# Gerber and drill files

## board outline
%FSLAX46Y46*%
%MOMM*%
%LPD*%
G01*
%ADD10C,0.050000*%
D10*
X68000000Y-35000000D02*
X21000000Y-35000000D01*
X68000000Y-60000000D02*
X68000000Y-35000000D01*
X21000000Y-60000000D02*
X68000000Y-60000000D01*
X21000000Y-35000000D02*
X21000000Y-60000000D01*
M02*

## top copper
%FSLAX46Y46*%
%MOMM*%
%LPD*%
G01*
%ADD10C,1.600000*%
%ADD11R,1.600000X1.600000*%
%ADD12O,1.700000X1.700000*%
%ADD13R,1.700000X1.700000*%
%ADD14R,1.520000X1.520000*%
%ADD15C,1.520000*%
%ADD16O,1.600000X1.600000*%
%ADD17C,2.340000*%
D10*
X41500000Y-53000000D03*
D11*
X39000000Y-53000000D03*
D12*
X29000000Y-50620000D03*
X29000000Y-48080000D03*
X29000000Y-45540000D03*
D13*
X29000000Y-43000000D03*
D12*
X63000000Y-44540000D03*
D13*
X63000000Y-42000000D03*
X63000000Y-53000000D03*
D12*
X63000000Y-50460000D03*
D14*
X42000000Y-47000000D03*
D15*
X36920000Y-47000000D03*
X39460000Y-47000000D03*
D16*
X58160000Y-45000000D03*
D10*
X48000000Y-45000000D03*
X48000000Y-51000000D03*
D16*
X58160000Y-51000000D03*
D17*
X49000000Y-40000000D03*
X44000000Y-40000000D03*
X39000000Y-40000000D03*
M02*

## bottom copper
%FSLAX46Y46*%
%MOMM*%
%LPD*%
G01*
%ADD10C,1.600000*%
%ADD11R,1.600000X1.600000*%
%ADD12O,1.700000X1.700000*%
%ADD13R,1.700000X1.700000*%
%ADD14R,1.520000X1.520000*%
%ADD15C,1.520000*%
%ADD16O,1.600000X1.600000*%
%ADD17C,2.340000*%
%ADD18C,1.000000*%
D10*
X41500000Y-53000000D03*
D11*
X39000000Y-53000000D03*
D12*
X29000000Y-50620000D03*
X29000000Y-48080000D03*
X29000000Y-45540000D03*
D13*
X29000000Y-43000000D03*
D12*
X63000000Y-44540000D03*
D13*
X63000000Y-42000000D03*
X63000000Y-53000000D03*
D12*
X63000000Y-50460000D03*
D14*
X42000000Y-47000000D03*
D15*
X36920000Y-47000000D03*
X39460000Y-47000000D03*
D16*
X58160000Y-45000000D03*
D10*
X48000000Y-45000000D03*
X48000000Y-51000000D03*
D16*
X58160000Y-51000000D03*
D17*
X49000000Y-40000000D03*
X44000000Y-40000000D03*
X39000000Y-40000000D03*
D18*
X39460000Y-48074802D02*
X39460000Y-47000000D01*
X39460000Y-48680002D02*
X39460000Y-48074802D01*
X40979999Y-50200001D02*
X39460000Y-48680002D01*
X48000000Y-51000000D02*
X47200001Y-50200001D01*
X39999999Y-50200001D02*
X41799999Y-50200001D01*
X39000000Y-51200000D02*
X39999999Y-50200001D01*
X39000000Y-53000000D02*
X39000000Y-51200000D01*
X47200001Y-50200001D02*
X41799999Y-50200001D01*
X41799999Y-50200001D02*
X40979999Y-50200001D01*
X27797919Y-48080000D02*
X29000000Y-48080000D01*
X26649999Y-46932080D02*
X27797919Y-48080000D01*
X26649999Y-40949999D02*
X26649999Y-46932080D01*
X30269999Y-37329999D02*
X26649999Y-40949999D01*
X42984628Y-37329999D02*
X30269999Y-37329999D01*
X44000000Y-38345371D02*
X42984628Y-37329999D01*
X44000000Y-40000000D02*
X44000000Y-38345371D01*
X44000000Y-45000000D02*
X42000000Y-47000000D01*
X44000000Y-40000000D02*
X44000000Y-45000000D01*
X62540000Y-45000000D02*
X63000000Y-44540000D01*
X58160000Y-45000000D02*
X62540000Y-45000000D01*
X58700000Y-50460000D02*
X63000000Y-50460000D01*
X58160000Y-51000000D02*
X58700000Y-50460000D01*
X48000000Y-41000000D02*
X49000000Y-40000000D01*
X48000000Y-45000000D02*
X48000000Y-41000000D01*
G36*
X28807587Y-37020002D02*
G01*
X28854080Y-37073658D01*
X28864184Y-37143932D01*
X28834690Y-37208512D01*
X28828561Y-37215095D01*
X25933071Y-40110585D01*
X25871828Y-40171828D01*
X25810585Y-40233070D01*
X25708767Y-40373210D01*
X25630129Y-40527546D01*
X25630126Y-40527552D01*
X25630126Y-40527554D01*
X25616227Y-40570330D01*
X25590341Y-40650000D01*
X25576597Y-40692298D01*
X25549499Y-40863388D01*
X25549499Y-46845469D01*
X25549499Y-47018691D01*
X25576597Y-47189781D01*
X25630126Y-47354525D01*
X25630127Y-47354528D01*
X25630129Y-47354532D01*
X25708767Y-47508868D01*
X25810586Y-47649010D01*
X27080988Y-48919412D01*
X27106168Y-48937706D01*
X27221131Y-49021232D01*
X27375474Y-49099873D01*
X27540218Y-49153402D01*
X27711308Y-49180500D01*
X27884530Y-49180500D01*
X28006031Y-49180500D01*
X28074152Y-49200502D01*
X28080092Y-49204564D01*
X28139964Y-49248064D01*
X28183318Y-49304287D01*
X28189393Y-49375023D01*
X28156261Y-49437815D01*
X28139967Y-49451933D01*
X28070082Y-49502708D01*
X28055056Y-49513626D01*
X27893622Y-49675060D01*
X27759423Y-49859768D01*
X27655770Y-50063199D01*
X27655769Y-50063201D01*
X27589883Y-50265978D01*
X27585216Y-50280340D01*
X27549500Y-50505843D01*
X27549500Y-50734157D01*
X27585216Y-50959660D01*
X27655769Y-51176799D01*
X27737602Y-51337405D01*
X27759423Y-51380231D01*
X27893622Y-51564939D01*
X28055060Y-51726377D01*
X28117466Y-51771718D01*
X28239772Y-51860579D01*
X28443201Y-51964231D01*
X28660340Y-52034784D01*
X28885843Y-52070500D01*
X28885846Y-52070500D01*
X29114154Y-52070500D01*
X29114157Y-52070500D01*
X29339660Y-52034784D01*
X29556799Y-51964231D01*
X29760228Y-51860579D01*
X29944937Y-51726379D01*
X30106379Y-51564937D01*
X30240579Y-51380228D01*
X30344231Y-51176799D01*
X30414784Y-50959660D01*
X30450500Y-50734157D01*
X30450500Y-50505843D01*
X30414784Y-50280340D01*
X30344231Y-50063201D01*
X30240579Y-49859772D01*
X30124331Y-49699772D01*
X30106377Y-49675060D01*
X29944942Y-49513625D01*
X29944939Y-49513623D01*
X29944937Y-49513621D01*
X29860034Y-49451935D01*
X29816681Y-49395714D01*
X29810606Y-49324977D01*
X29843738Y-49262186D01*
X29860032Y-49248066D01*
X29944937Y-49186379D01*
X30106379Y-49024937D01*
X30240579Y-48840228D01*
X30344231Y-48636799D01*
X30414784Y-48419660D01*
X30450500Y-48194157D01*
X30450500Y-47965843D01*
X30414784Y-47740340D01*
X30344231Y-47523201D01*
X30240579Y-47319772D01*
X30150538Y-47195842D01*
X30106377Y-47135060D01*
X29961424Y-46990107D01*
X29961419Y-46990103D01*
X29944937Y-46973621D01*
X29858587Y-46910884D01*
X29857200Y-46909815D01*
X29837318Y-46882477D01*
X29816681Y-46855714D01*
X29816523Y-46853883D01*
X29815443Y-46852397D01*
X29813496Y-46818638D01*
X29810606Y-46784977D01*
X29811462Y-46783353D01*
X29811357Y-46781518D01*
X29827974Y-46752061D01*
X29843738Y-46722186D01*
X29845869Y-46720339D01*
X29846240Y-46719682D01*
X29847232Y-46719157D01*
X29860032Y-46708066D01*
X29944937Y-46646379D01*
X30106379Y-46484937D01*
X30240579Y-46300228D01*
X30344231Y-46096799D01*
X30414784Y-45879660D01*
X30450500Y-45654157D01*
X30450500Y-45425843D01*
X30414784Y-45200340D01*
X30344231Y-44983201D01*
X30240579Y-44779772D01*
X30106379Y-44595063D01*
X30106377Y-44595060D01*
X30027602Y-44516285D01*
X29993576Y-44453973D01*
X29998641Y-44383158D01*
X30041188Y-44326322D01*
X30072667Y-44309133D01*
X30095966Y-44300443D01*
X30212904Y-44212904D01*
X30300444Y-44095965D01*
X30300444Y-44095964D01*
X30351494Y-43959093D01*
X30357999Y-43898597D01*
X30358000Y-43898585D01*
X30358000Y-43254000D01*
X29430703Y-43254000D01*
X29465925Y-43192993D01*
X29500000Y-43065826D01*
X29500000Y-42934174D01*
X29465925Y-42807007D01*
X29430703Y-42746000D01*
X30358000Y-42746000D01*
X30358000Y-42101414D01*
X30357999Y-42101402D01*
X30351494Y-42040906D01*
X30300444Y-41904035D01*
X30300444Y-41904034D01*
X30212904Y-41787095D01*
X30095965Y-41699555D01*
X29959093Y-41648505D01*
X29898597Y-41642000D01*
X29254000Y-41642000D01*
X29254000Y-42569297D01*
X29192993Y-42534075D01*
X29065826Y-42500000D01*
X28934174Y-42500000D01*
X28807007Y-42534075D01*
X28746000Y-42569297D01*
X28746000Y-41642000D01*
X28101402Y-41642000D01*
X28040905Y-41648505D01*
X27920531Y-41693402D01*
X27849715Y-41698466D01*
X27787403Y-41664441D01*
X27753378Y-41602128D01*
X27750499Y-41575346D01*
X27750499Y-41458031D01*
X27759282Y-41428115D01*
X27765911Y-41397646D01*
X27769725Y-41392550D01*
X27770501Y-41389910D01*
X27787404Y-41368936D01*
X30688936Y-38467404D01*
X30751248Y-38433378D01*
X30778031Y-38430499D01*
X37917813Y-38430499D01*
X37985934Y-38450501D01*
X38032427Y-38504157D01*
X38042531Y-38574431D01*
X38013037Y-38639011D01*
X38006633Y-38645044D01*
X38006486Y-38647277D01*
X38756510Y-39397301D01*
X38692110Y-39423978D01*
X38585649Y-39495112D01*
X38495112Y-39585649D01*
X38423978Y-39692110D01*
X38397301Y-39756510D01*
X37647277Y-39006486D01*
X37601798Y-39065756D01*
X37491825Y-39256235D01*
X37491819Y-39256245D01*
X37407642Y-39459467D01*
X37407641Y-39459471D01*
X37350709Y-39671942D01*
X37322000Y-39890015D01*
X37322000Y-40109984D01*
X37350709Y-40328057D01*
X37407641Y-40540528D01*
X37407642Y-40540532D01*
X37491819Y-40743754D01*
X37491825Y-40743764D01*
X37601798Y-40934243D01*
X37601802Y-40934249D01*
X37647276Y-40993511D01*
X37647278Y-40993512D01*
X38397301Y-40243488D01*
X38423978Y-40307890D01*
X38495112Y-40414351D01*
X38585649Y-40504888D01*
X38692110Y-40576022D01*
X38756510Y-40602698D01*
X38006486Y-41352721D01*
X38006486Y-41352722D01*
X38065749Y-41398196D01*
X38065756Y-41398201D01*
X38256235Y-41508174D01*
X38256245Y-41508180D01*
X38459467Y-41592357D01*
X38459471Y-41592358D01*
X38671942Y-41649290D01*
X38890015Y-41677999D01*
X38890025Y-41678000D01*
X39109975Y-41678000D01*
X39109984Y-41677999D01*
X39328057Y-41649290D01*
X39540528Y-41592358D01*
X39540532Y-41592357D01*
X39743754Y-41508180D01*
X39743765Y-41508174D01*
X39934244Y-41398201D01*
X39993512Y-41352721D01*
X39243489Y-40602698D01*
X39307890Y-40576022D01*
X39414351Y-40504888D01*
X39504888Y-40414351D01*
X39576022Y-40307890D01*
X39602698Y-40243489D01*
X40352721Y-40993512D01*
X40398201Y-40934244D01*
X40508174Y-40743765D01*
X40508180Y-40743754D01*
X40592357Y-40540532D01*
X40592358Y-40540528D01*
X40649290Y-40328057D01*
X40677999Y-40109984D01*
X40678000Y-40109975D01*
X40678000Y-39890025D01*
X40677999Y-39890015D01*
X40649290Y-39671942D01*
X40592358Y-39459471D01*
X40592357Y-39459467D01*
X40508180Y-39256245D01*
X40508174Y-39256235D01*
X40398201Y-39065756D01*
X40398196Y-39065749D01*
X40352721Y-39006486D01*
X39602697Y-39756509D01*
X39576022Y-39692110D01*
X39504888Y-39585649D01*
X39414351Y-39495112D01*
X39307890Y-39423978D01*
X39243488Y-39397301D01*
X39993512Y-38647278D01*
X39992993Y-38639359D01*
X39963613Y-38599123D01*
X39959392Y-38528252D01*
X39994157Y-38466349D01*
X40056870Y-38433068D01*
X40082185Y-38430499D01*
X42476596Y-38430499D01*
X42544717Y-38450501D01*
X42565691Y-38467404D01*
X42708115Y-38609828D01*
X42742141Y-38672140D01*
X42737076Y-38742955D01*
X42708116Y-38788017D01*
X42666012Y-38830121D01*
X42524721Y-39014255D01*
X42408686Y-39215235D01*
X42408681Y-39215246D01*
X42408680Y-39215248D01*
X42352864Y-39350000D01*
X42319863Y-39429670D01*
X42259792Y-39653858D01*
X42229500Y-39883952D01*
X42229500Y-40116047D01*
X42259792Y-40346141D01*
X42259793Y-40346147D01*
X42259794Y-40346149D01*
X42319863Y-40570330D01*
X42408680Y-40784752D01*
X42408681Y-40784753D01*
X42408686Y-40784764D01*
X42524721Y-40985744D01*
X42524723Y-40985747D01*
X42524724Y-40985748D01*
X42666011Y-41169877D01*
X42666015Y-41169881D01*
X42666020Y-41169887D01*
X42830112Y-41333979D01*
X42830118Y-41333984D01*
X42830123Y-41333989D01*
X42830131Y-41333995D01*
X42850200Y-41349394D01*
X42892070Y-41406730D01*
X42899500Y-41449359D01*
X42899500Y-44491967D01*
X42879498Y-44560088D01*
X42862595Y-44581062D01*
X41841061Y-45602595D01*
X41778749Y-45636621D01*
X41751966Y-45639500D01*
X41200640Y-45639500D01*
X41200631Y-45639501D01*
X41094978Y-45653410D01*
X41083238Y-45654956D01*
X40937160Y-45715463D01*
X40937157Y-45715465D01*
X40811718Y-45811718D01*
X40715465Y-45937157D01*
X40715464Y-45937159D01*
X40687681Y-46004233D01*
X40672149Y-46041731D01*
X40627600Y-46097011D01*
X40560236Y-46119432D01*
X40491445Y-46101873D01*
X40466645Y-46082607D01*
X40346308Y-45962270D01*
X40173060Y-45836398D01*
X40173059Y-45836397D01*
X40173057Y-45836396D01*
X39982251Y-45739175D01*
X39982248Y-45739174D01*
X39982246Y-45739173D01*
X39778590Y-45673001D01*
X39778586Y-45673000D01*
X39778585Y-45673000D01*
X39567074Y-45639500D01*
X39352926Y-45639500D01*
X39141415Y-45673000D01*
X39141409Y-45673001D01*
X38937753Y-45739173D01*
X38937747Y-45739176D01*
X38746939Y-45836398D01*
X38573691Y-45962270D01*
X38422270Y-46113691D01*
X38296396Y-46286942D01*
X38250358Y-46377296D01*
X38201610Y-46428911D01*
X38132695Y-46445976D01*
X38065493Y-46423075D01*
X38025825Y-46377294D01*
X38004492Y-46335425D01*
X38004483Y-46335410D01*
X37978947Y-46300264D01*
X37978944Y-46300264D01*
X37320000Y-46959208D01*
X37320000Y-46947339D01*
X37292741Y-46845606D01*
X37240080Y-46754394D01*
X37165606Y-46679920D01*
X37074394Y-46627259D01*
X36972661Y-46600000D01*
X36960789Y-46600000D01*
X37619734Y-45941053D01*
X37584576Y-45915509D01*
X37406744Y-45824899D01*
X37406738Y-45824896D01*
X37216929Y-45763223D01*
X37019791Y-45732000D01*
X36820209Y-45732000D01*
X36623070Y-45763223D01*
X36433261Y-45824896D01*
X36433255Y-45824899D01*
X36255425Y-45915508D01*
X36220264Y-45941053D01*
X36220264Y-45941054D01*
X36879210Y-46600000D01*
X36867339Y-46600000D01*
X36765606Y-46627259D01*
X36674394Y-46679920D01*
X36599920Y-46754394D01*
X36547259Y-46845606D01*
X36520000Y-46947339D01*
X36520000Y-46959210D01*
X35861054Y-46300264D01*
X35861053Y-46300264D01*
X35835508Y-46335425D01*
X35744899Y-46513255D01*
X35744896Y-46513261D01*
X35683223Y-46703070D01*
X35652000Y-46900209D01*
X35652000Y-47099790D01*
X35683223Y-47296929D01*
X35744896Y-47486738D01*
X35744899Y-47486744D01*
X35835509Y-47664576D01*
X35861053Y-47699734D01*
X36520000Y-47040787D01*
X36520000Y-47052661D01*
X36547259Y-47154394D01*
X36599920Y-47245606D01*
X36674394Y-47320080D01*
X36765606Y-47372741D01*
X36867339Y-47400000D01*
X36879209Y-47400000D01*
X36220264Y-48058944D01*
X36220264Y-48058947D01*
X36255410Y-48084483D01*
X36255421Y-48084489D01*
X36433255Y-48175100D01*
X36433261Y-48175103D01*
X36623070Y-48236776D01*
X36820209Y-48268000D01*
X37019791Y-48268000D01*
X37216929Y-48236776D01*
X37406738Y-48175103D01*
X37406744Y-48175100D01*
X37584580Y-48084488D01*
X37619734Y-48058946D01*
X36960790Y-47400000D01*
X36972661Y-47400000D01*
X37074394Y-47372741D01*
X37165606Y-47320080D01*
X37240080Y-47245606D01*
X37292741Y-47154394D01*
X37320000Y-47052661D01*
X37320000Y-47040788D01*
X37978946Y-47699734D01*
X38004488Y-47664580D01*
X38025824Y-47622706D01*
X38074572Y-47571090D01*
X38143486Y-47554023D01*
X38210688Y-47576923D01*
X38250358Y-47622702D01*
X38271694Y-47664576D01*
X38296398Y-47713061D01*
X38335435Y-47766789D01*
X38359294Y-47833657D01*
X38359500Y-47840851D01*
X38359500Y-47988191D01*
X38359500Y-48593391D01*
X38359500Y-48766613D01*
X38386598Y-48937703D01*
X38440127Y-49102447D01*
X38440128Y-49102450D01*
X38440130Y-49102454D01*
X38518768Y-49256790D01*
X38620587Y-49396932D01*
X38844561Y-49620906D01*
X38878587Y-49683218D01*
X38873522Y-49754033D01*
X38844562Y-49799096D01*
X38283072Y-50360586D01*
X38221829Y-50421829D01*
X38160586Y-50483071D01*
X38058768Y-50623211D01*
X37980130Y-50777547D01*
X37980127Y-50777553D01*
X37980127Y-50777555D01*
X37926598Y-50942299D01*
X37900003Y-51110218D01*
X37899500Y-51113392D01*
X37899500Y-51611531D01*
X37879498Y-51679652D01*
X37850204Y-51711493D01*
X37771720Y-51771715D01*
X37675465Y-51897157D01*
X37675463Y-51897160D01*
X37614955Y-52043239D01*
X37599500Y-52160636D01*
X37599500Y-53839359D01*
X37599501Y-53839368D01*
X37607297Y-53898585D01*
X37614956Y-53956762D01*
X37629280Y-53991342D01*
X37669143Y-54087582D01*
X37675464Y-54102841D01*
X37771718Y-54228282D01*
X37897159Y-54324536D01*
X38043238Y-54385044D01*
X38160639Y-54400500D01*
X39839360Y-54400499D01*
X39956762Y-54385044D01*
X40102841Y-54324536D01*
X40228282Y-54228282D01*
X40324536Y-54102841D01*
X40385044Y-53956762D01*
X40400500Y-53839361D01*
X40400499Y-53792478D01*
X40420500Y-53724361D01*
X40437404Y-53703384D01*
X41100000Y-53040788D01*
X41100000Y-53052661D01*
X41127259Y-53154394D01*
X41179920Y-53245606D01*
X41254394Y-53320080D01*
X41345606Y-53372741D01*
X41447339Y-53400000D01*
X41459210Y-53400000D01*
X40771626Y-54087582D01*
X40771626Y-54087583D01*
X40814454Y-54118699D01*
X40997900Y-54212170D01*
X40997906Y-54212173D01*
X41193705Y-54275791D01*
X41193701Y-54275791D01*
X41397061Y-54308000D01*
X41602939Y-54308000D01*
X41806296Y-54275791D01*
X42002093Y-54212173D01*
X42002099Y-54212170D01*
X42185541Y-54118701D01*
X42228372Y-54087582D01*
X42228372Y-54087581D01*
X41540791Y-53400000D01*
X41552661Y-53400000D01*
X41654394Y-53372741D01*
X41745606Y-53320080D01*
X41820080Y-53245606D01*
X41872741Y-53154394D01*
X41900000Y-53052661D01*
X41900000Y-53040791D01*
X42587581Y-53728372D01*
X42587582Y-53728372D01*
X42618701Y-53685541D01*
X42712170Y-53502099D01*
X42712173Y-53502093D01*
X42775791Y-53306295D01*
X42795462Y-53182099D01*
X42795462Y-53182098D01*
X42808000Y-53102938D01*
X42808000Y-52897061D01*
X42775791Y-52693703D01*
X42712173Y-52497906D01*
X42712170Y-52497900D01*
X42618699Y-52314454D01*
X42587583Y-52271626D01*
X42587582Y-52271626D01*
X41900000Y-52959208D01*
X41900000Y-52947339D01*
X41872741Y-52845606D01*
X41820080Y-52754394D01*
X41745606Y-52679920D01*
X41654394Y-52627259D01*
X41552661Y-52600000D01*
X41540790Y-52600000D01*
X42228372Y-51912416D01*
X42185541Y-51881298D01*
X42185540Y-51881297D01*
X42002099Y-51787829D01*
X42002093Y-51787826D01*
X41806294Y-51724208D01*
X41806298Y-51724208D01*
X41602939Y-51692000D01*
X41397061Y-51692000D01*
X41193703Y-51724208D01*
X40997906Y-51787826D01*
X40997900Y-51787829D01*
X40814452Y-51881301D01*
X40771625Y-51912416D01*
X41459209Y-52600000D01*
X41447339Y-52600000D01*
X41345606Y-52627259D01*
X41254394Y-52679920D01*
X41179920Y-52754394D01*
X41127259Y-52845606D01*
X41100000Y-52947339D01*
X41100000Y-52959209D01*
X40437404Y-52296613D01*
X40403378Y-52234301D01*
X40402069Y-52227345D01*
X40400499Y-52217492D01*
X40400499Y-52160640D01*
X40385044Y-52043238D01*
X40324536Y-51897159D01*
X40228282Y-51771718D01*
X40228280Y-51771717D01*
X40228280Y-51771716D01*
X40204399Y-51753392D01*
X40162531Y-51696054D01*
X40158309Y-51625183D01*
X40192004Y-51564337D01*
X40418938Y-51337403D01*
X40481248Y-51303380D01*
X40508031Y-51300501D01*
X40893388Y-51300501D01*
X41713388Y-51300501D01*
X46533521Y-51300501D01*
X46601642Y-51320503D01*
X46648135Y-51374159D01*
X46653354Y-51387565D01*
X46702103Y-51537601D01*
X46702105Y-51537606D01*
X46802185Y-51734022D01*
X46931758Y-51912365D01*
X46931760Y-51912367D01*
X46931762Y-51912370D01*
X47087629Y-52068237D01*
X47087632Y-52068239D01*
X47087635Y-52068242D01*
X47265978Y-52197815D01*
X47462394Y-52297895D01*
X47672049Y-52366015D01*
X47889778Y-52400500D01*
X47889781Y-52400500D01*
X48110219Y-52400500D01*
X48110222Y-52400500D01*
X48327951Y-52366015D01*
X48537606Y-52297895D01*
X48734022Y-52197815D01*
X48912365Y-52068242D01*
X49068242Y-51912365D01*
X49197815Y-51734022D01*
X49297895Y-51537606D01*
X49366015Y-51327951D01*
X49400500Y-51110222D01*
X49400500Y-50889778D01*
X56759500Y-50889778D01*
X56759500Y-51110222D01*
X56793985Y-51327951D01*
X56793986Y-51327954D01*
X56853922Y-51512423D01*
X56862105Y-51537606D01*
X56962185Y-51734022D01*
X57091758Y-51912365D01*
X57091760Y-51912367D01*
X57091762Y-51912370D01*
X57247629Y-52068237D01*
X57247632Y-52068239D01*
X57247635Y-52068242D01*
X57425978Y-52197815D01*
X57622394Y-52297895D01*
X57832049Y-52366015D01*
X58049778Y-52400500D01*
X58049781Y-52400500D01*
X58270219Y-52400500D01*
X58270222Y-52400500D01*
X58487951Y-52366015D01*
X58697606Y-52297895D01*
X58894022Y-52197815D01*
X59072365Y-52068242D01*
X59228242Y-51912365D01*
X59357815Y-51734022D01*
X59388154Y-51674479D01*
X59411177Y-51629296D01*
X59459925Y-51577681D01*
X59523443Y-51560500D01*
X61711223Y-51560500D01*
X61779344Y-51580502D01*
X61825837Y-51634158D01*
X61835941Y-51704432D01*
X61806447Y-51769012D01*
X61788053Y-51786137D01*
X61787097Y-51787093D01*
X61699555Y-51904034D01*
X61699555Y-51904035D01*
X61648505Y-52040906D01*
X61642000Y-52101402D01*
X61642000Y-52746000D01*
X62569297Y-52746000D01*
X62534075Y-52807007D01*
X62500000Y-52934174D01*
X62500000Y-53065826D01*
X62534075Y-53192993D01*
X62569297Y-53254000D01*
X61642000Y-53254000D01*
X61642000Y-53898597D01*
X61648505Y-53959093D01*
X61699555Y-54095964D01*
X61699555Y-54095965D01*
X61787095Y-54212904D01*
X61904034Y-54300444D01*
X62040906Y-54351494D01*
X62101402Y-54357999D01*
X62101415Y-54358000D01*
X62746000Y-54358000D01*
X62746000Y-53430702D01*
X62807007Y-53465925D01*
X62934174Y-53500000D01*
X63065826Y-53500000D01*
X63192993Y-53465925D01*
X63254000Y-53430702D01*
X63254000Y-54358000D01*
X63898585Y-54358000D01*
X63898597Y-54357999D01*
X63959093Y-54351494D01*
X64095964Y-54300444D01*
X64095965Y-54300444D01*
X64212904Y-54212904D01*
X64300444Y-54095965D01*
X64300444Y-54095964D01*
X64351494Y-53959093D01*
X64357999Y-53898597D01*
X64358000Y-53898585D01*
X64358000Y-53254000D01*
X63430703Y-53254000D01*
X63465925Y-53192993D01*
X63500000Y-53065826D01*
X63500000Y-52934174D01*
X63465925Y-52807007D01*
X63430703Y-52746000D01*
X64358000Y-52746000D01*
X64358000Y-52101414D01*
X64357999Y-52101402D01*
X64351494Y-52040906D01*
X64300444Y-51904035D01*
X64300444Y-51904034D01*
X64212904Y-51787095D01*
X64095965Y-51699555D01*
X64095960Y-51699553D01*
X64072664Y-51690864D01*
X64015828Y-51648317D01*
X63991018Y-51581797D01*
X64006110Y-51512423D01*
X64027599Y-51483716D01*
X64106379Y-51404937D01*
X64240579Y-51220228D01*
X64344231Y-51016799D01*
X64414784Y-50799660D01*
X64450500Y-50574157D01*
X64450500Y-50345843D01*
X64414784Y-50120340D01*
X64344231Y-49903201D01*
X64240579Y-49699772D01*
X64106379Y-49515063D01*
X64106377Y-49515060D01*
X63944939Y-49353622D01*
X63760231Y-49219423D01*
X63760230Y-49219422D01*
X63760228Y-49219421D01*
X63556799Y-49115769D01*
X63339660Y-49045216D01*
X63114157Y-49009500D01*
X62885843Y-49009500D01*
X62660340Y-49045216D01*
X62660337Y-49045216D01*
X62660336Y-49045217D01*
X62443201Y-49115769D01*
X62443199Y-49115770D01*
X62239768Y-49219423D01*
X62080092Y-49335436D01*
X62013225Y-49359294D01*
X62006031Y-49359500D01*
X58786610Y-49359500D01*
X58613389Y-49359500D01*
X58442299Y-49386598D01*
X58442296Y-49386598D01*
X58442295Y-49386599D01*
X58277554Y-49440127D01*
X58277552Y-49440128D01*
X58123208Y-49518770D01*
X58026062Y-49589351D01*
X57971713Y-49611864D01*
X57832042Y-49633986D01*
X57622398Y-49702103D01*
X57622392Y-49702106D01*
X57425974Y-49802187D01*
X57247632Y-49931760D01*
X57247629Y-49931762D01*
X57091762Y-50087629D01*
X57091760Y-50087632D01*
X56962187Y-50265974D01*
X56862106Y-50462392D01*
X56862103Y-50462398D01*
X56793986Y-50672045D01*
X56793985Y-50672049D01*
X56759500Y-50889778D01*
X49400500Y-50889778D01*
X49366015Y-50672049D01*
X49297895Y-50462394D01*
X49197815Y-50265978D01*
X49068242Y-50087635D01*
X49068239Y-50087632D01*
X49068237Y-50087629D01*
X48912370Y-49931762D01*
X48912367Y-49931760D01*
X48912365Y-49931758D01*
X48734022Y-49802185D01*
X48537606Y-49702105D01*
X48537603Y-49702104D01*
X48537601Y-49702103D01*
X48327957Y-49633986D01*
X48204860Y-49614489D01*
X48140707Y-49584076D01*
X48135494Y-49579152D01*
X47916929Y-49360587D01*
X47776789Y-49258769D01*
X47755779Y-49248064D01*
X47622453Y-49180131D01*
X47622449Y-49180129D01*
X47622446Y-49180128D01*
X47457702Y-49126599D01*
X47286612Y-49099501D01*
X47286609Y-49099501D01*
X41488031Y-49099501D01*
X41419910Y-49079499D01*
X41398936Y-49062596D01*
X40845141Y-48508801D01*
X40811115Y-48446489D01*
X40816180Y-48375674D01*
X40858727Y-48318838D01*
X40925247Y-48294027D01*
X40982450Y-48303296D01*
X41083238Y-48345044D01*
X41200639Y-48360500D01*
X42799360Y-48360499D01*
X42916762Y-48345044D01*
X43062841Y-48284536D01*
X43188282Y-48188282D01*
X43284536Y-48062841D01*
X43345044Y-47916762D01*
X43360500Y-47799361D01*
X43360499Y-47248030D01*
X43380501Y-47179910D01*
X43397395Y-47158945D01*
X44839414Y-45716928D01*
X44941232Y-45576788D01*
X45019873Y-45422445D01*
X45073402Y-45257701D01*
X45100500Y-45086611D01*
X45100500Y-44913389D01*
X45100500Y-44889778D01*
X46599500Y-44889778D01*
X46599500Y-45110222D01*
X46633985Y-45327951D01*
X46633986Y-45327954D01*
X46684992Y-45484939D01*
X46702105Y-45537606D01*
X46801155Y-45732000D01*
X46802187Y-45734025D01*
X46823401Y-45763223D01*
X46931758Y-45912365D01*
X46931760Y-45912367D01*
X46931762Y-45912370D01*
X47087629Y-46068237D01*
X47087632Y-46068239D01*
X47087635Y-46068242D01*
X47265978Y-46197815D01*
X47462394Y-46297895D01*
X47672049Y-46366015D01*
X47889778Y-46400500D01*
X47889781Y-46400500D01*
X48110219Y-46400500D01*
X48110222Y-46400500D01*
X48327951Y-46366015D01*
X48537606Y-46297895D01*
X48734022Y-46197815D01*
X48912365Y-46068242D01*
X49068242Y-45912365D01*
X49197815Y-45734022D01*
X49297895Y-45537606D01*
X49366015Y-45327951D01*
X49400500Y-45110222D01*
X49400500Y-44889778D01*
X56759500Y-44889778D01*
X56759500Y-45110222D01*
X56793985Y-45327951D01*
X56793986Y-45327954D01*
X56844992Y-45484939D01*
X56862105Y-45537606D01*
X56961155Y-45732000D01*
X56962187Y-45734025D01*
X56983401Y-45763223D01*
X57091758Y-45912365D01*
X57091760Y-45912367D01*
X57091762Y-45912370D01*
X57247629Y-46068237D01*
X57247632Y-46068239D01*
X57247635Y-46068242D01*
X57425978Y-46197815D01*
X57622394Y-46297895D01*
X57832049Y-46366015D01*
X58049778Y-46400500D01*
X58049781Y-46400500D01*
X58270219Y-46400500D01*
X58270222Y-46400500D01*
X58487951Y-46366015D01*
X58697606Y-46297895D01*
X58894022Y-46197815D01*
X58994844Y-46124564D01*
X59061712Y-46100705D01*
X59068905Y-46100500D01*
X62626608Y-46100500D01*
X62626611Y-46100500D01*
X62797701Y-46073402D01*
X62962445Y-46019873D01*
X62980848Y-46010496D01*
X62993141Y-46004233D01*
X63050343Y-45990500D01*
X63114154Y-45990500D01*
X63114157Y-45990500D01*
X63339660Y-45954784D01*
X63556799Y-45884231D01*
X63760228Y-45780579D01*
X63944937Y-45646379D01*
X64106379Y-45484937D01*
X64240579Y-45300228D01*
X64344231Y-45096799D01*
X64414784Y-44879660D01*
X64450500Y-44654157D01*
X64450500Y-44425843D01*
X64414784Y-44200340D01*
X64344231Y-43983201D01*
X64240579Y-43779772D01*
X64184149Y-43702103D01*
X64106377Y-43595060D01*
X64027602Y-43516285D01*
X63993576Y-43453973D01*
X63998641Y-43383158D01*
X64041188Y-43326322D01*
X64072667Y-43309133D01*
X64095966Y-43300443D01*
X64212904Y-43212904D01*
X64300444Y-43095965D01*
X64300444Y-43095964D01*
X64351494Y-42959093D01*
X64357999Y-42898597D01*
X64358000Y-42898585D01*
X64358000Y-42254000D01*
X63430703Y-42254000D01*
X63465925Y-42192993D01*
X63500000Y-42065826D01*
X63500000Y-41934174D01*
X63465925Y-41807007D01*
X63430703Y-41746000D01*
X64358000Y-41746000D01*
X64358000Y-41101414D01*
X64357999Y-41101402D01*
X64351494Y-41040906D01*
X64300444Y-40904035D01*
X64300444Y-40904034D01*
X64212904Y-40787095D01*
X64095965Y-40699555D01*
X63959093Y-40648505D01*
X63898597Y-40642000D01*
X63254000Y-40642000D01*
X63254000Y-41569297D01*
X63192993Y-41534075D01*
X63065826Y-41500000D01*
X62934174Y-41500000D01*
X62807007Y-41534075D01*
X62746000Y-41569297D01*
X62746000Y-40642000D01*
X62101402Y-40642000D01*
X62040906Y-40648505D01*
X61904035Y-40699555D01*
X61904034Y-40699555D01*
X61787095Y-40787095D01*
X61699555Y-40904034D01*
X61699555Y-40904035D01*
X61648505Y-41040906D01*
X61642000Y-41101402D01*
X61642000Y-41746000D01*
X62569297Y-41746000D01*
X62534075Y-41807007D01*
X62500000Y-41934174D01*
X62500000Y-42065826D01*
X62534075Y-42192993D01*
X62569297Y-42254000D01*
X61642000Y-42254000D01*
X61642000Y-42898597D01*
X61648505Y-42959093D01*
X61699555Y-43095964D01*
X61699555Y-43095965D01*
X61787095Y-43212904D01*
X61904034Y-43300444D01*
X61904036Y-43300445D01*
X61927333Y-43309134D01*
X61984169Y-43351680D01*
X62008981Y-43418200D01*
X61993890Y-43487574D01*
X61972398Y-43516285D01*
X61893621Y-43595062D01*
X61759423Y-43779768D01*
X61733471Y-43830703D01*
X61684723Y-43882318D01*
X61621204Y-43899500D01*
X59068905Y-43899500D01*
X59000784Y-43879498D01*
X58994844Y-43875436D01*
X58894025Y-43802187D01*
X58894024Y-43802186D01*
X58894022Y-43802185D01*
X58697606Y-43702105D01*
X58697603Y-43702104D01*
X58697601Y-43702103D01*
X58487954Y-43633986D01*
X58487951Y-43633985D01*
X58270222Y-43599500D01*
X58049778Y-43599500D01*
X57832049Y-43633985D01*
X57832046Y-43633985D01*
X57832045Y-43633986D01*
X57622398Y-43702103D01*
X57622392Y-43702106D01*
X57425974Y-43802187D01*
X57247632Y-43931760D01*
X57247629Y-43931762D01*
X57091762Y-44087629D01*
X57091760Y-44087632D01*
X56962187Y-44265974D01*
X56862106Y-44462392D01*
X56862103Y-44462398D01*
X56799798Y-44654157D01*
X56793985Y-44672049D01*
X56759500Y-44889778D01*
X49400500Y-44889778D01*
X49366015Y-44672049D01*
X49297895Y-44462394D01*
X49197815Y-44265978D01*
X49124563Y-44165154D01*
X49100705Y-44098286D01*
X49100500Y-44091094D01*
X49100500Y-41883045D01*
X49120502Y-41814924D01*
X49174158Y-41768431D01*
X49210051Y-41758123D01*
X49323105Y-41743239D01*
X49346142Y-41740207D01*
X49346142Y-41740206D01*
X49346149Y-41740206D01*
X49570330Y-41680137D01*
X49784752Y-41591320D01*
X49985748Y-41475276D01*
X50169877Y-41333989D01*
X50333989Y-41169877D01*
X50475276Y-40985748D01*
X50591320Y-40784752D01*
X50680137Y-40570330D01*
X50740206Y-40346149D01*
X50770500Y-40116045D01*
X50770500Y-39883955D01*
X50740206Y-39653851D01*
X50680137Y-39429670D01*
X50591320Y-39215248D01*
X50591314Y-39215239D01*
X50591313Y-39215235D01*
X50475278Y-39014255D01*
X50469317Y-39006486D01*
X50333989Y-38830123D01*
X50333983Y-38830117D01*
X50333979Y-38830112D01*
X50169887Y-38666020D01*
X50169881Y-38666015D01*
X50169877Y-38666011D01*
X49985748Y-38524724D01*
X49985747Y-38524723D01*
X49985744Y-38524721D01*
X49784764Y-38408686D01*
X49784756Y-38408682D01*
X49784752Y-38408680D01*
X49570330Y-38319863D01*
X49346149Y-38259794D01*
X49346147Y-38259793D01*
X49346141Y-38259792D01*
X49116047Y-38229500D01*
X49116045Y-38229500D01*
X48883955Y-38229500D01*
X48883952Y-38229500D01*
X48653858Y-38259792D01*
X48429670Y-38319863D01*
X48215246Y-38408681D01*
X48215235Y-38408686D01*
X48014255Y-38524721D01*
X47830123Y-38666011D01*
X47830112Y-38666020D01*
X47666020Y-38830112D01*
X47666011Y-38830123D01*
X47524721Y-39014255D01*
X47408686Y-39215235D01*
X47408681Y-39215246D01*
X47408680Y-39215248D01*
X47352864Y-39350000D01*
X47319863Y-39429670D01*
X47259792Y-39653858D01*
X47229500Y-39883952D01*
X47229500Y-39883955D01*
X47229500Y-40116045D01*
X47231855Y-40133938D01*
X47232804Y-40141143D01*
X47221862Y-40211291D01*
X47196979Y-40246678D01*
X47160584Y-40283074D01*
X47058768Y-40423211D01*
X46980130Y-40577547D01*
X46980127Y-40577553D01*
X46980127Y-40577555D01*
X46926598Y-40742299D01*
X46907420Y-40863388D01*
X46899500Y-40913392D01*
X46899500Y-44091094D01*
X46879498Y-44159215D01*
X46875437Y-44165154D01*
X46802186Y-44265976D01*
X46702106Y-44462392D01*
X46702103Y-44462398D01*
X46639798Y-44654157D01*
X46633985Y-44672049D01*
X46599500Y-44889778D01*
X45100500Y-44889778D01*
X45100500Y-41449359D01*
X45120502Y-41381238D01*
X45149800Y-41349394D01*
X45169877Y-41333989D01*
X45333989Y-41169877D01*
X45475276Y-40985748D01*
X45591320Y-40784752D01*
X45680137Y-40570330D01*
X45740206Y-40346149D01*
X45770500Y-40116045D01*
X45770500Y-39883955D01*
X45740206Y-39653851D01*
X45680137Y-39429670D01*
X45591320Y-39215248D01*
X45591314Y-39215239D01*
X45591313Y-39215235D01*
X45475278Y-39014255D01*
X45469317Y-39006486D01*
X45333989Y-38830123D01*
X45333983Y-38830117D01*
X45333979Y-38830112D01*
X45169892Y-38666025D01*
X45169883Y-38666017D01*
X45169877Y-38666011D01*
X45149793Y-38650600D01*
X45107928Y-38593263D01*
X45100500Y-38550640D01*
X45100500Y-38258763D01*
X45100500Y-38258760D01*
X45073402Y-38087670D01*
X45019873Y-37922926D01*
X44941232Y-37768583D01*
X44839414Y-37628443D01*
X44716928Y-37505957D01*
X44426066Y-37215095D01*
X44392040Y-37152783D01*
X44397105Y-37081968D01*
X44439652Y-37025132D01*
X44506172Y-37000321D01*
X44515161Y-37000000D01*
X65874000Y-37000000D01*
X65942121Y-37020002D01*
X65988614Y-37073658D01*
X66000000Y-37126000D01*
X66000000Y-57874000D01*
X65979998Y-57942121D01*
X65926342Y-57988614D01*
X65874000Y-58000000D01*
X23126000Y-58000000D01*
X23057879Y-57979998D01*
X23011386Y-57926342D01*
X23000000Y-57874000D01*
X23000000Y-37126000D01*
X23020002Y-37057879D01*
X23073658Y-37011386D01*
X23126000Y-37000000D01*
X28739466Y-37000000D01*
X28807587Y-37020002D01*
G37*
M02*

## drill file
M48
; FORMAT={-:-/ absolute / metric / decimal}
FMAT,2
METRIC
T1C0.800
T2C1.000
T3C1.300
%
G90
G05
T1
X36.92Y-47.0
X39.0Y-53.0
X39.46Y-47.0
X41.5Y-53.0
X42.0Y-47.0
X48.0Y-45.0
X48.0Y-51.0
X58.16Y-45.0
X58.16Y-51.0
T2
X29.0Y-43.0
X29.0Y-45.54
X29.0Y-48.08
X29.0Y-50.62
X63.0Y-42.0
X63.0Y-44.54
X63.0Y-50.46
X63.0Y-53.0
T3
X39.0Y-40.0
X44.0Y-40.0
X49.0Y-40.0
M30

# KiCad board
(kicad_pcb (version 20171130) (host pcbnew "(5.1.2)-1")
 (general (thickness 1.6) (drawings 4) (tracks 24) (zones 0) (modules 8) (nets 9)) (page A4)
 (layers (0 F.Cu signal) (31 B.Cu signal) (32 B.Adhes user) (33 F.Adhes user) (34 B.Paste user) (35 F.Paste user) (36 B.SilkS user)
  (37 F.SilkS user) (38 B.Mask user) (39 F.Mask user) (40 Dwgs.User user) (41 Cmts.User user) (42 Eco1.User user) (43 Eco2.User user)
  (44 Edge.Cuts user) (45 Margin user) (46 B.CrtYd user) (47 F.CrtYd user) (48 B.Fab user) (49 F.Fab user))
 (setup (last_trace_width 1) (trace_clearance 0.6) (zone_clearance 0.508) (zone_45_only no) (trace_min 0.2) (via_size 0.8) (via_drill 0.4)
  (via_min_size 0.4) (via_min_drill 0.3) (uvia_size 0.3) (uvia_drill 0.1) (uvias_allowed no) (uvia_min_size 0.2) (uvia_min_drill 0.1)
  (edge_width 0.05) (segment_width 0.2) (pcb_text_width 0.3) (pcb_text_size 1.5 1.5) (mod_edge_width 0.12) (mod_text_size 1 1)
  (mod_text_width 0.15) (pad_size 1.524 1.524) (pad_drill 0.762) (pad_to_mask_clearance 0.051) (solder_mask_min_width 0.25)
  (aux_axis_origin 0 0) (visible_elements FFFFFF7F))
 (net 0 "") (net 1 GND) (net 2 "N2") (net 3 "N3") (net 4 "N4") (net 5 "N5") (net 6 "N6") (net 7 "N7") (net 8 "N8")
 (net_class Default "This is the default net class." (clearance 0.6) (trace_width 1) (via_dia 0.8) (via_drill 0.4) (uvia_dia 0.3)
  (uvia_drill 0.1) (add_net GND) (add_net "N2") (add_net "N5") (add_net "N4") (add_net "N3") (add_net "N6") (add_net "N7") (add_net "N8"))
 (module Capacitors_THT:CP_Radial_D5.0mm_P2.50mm (layer F.Cu) (at 39 53)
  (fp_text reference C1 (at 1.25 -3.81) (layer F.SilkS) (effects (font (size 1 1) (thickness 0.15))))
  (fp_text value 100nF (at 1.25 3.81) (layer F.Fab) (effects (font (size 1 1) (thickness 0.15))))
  (pad 2 thru_hole circle (at 2.5 0) (size 1.6 1.6) (drill 0.8) (layers *.Cu *.Mask) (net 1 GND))
  (pad 1 thru_hole rect (at 0 0) (size 1.6 1.6) (drill 0.8) (layers *.Cu *.Mask) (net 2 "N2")))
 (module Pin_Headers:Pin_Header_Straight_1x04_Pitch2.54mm (layer F.Cu) (at 29 43)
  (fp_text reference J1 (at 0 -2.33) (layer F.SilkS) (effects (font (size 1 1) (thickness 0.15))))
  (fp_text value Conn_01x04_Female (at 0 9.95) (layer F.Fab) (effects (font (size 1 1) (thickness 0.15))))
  (pad 4 thru_hole oval (at 0 7.62) (size 1.7 1.7) (drill 1) (layers *.Cu *.Mask) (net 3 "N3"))
  (pad 3 thru_hole oval (at 0 5.08) (size 1.7 1.7) (drill 1) (layers *.Cu *.Mask) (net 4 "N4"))
  (pad 2 thru_hole oval (at 0 2.54) (size 1.7 1.7) (drill 1) (layers *.Cu *.Mask) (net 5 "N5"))
  (pad 1 thru_hole rect (at 0 0) (size 1.7 1.7) (drill 1) (layers *.Cu *.Mask) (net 1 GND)))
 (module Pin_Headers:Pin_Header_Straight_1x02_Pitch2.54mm (layer F.Cu) (at 63 42)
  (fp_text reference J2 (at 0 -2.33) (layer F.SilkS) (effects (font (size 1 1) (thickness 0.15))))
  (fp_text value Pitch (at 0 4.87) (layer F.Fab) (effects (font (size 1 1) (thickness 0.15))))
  (pad 2 thru_hole oval (at 0 2.54) (size 1.7 1.7) (drill 1) (layers *.Cu *.Mask) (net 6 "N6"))
  (pad 1 thru_hole rect (at 0 0) (size 1.7 1.7) (drill 1) (layers *.Cu *.Mask) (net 1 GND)))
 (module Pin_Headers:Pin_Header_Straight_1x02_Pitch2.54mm (layer F.Cu) (at 63 53 180)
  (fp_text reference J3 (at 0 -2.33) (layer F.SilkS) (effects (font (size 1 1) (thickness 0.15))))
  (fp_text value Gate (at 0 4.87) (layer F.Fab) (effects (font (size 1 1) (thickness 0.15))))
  (pad 1 thru_hole rect (at 0 0 180) (size 1.7 1.7) (drill 1) (layers *.Cu *.Mask) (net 1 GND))
  (pad 2 thru_hole oval (at 0 2.54 180) (size 1.7 1.7) (drill 1) (layers *.Cu *.Mask) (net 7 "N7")))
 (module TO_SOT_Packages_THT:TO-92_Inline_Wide (layer F.Cu) (at 42 47 180)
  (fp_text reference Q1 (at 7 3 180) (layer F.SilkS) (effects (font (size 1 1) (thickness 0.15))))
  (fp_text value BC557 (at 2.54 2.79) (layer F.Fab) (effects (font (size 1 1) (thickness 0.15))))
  (pad 1 thru_hole rect (at 0 0 270) (size 1.52 1.52) (drill 0.8) (layers *.Cu *.Mask) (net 4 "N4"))
  (pad 3 thru_hole circle (at 5.08 0 270) (size 1.52 1.52) (drill 0.8) (layers *.Cu *.Mask) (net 1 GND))
  (pad 2 thru_hole circle (at 2.54 0 270) (size 1.52 1.52) (drill 0.8) (layers *.Cu *.Mask) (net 2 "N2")))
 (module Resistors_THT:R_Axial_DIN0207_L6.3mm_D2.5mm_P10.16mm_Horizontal (layer F.Cu) (at 48 45)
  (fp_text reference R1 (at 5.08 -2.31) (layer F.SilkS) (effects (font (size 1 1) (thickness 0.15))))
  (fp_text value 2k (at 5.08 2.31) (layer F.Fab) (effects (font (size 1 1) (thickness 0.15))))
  (pad 2 thru_hole oval (at 10.16 0) (size 1.6 1.6) (drill 0.8) (layers *.Cu *.Mask) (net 6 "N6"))
  (pad 1 thru_hole circle (at 0 0) (size 1.6 1.6) (drill 0.8) (layers *.Cu *.Mask) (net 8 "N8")))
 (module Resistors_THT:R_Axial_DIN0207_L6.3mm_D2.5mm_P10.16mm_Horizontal (layer F.Cu) (at 48 51)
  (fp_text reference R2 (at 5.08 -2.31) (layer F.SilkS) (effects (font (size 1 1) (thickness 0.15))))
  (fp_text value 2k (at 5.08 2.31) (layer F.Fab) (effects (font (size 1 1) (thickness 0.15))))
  (pad 1 thru_hole circle (at 0 0) (size 1.6 1.6) (drill 0.8) (layers *.Cu *.Mask) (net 2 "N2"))
  (pad 2 thru_hole oval (at 10.16 0) (size 1.6 1.6) (drill 0.8) (layers *.Cu *.Mask) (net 7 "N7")))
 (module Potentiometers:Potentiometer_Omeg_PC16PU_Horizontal (layer F.Cu) (at 49 40 90)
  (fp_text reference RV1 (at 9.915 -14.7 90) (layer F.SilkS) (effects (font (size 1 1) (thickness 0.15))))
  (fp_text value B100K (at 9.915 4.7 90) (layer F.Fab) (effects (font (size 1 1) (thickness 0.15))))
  (pad 1 thru_hole circle (at 0 0 90) (size 2.34 2.34) (drill 1.3) (layers *.Cu *.Mask) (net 8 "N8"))
  (pad 2 thru_hole circle (at 0 -5 90) (size 2.34 2.34) (drill 1.3) (layers *.Cu *.Mask) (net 4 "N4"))
  (pad 3 thru_hole circle (at 0 -10 90) (size 2.34 2.34) (drill 1.3) (layers *.Cu *.Mask) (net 1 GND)))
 (gr_line (start 68 35) (end 21 35) (layer Edge.Cuts) (width 0.05))
 (gr_line (start 68 60) (end 68 35) (layer Edge.Cuts) (width 0.05))
 (gr_line (start 21 60) (end 68 60) (layer Edge.Cuts) (width 0.05))
 (gr_line (start 21 35) (end 21 60) (layer Edge.Cuts) (width 0.05))
 (segment (start 39.46 48.074802) (end 39.46 47) (width 1) (layer B.Cu) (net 2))
 (segment (start 39.46 48.680002) (end 39.46 48.074802) (width 1) (layer B.Cu) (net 2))
 (segment (start 40.979999 50.200001) (end 39.46 48.680002) (width 1) (layer B.Cu) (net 2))
 (segment (start 48 51) (end 47.200001 50.200001) (width 1) (layer B.Cu) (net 2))
 (segment (start 39.999999 50.200001) (end 41.799999 50.200001) (width 1) (layer B.Cu) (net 2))
 (segment (start 39 51.2) (end 39.999999 50.200001) (width 1) (layer B.Cu) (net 2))
 (segment (start 39 53) (end 39 51.2) (width 1) (layer B.Cu) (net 2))
 (segment (start 47.200001 50.200001) (end 41.799999 50.200001) (width 1) (layer B.Cu) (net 2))
 (segment (start 41.799999 50.200001) (end 40.979999 50.200001) (width 1) (layer B.Cu) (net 2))
 (segment (start 27.797919 48.08) (end 29 48.08) (width 1) (layer B.Cu) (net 4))
 (segment (start 26.649999 46.93208) (end 27.797919 48.08) (width 1) (layer B.Cu) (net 4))
 (segment (start 26.649999 40.949999) (end 26.649999 46.93208) (width 1) (layer B.Cu) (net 4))
 (segment (start 30.269999 37.329999) (end 26.649999 40.949999) (width 1) (layer B.Cu) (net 4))
 (segment (start 42.984628 37.329999) (end 30.269999 37.329999) (width 1) (layer B.Cu) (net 4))
 (segment (start 44 38.345371) (end 42.984628 37.329999) (width 1) (layer B.Cu) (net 4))
 (segment (start 44 40) (end 44 38.345371) (width 1) (layer B.Cu) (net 4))
 (segment (start 44 45) (end 42 47) (width 1) (layer B.Cu) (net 4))
 (segment (start 44 40) (end 44 45) (width 1) (layer B.Cu) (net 4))
 (segment (start 62.54 45) (end 63 44.54) (width 1) (layer B.Cu) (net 6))
 (segment (start 58.16 45) (end 62.54 45) (width 1) (layer B.Cu) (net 6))
 (segment (start 58.7 50.46) (end 63 50.46) (width 1) (layer B.Cu) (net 7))
 (segment (start 58.16 51) (end 58.7 50.46) (width 1) (layer B.Cu) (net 7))
 (segment (start 48 41) (end 49 40) (width 1) (layer B.Cu) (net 8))
 (segment (start 48 45) (end 48 41) (width 1) (layer B.Cu) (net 8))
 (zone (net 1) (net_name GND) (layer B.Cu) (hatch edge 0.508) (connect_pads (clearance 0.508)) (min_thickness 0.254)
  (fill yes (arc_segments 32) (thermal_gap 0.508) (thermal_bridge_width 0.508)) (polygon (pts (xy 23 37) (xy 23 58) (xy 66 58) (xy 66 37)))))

